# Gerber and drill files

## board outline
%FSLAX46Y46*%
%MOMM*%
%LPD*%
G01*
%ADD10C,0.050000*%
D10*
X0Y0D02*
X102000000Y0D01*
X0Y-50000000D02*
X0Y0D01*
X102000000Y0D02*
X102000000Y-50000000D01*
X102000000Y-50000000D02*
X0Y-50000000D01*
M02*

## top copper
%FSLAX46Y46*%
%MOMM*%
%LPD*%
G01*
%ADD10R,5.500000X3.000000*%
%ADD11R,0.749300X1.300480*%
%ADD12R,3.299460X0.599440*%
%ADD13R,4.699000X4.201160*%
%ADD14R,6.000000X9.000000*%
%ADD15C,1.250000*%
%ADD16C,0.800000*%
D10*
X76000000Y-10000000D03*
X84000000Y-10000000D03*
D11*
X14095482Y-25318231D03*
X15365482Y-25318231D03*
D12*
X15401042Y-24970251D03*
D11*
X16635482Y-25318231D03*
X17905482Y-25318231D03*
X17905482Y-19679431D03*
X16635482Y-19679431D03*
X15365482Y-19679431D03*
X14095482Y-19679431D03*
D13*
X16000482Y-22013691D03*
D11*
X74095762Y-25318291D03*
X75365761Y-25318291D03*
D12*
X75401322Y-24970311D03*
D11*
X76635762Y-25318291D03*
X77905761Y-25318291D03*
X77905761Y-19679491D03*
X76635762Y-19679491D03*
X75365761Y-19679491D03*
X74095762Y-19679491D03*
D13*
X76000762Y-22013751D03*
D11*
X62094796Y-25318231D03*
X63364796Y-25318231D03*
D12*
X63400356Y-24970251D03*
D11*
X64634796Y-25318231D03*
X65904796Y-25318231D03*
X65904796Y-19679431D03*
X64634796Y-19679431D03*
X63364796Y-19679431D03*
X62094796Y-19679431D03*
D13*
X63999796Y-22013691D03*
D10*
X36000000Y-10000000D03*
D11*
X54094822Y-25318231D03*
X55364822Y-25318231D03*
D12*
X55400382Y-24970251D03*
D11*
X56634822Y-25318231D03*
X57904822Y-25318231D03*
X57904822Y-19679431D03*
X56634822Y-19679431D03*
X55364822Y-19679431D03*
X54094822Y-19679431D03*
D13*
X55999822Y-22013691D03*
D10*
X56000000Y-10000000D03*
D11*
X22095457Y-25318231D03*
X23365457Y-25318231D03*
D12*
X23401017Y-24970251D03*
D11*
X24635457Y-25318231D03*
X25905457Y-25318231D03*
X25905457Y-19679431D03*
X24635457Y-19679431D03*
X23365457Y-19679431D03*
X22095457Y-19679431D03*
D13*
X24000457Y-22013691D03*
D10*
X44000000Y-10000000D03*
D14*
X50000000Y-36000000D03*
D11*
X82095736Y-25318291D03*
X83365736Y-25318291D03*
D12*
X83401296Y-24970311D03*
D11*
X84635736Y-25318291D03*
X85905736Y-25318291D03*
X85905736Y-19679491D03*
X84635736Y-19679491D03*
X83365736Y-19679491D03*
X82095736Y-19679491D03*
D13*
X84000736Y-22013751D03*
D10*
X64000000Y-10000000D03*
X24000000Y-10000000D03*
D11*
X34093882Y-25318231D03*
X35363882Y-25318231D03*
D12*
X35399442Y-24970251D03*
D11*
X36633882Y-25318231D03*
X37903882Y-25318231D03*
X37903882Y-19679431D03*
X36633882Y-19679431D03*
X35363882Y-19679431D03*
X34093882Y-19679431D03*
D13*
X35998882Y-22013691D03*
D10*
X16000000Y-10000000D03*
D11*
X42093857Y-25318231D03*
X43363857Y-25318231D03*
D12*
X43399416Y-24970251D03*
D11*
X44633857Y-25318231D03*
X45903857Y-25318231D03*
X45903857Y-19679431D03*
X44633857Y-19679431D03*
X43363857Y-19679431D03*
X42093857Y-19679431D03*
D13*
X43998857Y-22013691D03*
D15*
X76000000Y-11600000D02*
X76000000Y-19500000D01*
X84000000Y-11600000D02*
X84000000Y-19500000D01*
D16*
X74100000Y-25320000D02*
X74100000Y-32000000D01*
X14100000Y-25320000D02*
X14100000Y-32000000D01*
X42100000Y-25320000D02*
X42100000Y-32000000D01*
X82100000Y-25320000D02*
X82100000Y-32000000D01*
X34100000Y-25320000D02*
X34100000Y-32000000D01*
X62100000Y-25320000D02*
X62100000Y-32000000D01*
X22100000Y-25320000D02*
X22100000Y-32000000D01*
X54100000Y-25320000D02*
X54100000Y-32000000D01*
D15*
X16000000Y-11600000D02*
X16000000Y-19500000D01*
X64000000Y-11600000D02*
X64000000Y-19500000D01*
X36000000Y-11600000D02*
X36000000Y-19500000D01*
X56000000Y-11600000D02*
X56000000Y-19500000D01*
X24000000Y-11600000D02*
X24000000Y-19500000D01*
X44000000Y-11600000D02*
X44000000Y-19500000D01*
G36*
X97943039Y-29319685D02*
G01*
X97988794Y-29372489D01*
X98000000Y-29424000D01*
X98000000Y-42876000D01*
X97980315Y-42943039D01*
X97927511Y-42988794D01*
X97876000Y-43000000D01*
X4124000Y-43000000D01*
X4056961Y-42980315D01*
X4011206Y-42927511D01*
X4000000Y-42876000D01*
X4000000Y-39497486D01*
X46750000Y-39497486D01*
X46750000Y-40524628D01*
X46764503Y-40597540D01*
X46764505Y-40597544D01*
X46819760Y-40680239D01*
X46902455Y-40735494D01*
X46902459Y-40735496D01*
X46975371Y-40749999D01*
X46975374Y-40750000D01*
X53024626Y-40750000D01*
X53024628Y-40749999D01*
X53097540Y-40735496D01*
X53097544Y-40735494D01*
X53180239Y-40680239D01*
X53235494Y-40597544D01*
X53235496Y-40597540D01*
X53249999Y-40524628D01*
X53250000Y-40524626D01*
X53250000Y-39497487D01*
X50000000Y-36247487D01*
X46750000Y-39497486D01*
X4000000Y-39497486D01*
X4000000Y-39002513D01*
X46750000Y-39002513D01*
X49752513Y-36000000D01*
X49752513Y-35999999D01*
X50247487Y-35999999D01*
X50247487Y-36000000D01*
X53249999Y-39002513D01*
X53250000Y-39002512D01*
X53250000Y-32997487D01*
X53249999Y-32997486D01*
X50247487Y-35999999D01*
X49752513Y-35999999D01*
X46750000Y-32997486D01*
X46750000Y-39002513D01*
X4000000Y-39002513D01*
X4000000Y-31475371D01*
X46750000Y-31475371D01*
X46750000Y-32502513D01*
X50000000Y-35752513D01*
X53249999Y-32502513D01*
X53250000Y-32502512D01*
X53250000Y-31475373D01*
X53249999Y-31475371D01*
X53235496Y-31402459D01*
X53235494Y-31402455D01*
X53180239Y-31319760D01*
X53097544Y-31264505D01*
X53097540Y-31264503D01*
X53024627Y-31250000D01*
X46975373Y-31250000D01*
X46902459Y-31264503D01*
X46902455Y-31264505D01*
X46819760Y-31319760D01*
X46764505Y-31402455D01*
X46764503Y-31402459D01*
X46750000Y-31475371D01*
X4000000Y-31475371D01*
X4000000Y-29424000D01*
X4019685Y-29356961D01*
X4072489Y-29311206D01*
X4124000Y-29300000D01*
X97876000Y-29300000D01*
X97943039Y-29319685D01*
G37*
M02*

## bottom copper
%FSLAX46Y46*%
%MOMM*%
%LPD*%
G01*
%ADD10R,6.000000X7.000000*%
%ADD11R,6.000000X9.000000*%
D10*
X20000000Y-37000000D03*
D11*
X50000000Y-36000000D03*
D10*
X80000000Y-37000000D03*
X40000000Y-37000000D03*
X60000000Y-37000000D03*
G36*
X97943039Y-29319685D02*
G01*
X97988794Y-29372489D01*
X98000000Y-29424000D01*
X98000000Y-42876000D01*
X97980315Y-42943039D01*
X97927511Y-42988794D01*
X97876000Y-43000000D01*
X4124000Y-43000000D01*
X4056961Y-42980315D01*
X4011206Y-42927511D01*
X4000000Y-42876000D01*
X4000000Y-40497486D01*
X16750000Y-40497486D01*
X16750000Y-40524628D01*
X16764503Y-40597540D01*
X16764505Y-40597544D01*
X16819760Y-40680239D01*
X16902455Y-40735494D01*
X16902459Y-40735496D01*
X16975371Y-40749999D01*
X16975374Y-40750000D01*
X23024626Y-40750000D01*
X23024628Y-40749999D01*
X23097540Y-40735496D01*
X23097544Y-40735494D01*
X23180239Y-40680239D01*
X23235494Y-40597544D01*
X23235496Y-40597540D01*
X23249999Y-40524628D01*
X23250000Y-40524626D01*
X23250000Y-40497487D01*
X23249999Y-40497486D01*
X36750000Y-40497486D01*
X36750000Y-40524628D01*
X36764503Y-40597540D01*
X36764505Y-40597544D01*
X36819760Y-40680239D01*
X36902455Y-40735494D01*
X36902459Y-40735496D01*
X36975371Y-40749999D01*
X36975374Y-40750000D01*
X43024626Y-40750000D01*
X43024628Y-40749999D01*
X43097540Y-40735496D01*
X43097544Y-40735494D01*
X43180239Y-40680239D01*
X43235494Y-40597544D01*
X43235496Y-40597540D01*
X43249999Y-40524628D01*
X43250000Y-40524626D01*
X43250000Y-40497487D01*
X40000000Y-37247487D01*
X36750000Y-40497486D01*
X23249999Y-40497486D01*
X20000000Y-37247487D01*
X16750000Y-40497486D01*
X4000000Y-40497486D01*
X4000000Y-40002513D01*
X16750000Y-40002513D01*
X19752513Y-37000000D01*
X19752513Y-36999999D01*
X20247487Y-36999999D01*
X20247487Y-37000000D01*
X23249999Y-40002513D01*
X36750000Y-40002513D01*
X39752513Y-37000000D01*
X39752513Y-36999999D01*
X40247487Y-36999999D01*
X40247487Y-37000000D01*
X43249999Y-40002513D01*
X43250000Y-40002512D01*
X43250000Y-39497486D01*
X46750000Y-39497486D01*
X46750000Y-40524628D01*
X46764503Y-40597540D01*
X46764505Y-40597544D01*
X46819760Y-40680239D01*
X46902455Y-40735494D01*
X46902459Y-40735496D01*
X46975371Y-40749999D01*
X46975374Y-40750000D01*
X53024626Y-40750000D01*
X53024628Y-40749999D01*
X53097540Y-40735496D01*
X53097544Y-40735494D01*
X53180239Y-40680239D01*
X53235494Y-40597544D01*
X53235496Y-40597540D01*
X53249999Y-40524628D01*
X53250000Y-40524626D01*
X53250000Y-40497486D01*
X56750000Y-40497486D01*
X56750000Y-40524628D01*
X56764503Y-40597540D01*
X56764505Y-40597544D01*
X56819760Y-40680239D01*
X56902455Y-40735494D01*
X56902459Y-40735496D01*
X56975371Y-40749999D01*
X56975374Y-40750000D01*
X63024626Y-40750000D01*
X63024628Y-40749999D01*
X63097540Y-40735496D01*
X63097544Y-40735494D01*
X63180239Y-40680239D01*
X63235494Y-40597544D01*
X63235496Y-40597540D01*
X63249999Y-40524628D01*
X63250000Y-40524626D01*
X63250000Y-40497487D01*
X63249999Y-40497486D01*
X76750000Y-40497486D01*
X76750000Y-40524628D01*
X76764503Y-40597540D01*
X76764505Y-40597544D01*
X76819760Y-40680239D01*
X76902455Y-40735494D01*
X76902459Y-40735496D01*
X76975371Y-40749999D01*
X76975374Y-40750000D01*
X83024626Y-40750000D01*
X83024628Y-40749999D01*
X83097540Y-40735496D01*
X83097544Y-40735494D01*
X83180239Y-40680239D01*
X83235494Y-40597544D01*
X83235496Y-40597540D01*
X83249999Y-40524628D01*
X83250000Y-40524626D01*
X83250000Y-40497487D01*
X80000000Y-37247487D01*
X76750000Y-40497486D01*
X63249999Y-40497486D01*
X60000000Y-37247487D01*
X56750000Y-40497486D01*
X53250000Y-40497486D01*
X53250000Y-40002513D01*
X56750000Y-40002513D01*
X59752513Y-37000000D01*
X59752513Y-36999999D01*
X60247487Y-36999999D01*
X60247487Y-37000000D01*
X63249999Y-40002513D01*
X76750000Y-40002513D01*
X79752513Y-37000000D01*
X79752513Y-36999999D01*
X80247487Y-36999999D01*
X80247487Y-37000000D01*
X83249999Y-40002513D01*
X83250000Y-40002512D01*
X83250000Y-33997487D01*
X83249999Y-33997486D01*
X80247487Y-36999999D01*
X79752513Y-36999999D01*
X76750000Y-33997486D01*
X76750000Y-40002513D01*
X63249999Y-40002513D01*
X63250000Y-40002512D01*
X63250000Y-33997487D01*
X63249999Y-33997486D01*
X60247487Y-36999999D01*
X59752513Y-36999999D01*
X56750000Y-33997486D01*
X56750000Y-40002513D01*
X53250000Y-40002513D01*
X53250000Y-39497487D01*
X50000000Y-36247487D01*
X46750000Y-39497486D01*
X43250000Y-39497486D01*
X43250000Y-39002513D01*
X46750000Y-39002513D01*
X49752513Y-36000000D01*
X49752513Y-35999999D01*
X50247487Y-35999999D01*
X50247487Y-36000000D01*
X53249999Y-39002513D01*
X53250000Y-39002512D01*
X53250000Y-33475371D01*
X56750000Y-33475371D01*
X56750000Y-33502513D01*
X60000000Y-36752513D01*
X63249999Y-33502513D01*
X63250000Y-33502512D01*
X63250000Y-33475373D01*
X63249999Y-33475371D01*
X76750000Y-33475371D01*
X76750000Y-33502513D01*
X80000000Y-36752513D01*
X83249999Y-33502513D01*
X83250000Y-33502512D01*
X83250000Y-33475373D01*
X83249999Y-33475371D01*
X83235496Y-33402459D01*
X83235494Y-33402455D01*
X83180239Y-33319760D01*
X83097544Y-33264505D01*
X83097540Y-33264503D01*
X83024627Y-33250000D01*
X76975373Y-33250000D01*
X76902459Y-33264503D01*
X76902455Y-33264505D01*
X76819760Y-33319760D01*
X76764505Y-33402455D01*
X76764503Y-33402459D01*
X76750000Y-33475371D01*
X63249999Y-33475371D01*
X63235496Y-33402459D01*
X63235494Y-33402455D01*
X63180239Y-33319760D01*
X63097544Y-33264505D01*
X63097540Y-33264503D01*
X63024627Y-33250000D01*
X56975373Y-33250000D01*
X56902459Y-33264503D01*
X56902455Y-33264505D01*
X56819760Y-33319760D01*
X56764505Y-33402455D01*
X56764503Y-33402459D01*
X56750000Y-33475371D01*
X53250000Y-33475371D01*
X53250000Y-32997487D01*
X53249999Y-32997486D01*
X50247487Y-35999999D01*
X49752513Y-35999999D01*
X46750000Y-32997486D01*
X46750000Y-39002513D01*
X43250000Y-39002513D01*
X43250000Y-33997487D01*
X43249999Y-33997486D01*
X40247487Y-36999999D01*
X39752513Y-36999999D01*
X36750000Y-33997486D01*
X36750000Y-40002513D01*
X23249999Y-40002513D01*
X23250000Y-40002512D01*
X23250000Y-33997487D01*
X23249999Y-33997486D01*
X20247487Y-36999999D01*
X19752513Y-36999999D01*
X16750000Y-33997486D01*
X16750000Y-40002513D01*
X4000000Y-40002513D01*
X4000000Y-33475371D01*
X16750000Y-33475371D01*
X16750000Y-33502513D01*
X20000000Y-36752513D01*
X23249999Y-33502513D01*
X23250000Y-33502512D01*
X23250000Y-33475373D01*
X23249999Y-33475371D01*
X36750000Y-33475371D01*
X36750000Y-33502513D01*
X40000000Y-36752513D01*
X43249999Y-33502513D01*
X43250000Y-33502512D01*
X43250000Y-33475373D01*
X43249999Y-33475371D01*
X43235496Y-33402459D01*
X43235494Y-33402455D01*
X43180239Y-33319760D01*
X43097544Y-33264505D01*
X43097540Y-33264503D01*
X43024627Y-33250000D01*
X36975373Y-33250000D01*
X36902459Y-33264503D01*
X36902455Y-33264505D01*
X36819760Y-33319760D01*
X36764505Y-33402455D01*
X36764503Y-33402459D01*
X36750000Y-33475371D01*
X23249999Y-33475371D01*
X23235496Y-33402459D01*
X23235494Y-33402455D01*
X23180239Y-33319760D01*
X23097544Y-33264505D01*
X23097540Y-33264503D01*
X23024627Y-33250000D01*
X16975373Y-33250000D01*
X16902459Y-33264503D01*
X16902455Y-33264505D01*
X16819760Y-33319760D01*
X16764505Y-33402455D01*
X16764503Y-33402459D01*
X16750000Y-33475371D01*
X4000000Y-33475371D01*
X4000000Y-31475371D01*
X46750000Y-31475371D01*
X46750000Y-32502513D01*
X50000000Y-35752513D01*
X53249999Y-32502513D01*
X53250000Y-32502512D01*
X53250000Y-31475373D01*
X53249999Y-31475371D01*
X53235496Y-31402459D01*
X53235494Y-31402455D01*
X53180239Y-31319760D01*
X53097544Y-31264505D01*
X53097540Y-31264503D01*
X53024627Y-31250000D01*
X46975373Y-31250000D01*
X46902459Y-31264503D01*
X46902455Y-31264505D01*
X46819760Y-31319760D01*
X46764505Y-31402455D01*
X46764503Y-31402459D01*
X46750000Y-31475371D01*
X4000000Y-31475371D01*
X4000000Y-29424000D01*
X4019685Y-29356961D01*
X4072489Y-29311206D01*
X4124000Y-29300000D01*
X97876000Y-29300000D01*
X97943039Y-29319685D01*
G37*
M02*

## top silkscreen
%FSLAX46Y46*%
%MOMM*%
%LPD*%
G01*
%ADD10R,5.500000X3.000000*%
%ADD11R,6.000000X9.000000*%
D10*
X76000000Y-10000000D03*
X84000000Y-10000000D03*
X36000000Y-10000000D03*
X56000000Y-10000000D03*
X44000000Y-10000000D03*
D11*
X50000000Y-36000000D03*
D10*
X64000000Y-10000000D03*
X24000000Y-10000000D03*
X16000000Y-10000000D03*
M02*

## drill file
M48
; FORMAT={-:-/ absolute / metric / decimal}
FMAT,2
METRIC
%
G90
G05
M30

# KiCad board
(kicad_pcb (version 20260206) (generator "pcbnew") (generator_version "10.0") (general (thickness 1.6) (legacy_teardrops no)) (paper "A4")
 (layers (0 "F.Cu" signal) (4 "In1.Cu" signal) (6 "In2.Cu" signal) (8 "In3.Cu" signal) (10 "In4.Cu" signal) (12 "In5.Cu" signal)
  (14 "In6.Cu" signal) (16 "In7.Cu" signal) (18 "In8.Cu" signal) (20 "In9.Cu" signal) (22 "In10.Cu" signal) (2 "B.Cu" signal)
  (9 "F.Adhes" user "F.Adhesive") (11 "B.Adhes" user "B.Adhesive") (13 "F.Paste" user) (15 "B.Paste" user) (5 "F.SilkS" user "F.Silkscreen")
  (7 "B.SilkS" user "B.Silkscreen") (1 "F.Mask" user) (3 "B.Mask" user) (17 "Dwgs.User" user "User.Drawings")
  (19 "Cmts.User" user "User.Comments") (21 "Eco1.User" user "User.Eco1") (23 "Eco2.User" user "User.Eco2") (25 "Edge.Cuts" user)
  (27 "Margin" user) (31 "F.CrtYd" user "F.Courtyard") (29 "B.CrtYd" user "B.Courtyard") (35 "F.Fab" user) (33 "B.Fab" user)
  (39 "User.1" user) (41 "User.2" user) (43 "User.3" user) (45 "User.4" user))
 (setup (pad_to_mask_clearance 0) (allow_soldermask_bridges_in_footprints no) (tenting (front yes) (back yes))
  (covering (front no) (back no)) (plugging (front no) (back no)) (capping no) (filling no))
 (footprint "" (layer "F.Cu") (at 76 10)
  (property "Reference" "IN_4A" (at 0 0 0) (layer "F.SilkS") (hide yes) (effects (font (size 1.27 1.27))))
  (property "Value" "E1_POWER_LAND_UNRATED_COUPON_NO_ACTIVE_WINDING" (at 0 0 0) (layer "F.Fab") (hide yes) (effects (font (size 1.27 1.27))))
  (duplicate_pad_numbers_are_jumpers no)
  (pad "1" smd rect (at 0 0) (size 5.5 3)
   (layers "F.Cu" "F.Mask" "F.SilkS" "F.Adhes" "F.Paste" "F.CrtYd" "F.Fab") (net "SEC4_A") (thermal_bridge_angle 45)))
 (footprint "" (layer "F.Cu") (at 84 10)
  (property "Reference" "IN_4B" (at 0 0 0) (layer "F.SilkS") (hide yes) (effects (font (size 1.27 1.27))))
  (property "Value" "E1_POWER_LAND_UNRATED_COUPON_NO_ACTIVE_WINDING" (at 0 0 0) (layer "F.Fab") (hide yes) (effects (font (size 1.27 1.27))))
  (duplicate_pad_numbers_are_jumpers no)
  (pad "1" smd rect (at 0 0) (size 5.5 3)
   (layers "F.Cu" "F.Mask" "F.SilkS" "F.Adhes" "F.Paste" "F.CrtYd" "F.Fab") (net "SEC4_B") (thermal_bridge_angle 45)))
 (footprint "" (layer "F.Cu") (at 16 22.5)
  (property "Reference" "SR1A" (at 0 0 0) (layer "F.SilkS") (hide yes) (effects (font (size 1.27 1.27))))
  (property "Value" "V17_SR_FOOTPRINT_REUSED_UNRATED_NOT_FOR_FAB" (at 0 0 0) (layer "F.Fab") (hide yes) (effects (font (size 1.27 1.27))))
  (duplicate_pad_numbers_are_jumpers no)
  (pad "1" smd rect (at -1.904518 2.818231 90) (size 1.30048 0.7493) (layers "F.Cu" "F.Mask" "F.Paste") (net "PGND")
   (thermal_bridge_angle 45))
  (pad "2" smd rect (at -0.634518 2.818231 90) (size 1.30048 0.7493) (layers "F.Cu" "F.Mask" "F.Paste") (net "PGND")
   (thermal_bridge_angle 45))
  (pad "3" smd rect (at -0.598958 2.470251 90) (size 0.59944 3.29946) (layers "F.Cu" "F.Mask" "F.Paste") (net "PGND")
   (thermal_bridge_angle 45))
  (pad "3" smd rect (at 0.635482 2.818231 90) (size 1.30048 0.7493) (layers "F.Cu" "F.Mask" "F.Paste") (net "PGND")
   (thermal_bridge_angle 45))
  (pad "4" smd rect (at 1.905482 2.818231 90) (size 1.30048 0.7493) (layers "F.Cu" "F.Mask" "F.Paste") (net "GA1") (thermal_bridge_angle 45))
  (pad "5" smd rect (at 1.905482 -2.820569 270) (size 1.30048 0.7493) (layers "F.Cu" "F.Mask" "F.Paste") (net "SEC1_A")
   (thermal_bridge_angle 45))
  (pad "6" smd rect (at 0.635482 -2.820569 270) (size 1.30048 0.7493) (layers "F.Cu" "F.Mask" "F.Paste") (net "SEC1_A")
   (thermal_bridge_angle 45))
  (pad "7" smd rect (at -0.634518 -2.820569 270) (size 1.30048 0.7493) (layers "F.Cu" "F.Mask" "F.Paste") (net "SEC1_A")
   (thermal_bridge_angle 45))
  (pad "8" smd rect (at -1.904518 -2.820569 270) (size 1.30048 0.7493) (layers "F.Cu" "F.Mask" "F.Paste") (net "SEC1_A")
   (thermal_bridge_angle 45))
  (pad "8" smd rect (at 0.000482 -0.486309) (size 4.699 4.20116) (layers "F.Cu" "F.Mask" "F.Paste") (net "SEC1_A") (thermal_bridge_angle 45)))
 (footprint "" (layer "F.Cu") (at 76 22.5)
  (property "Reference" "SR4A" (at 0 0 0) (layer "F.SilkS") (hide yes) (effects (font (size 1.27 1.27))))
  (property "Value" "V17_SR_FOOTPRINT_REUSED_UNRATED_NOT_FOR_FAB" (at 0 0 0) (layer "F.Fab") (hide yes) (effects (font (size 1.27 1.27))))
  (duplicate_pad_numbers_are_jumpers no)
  (pad "1" smd rect (at -1.904238 2.818291 90) (size 1.30048 0.7493) (layers "F.Cu" "F.Mask" "F.Paste") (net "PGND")
   (thermal_bridge_angle 45))
  (pad "2" smd rect (at -0.634239 2.818291 90) (size 1.30048 0.7493) (layers "F.Cu" "F.Mask" "F.Paste") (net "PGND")
   (thermal_bridge_angle 45))
  (pad "3" smd rect (at -0.598678 2.470311 90) (size 0.59944 3.29946) (layers "F.Cu" "F.Mask" "F.Paste") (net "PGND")
   (thermal_bridge_angle 45))
  (pad "3" smd rect (at 0.635762 2.818291 90) (size 1.30048 0.7493) (layers "F.Cu" "F.Mask" "F.Paste") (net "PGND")
   (thermal_bridge_angle 45))
  (pad "4" smd rect (at 1.905761 2.818291 90) (size 1.30048 0.7493) (layers "F.Cu" "F.Mask" "F.Paste") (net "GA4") (thermal_bridge_angle 45))
  (pad "5" smd rect (at 1.905761 -2.820509 270) (size 1.30048 0.7493) (layers "F.Cu" "F.Mask" "F.Paste") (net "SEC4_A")
   (thermal_bridge_angle 45))
  (pad "6" smd rect (at 0.635762 -2.820509 270) (size 1.30048 0.7493) (layers "F.Cu" "F.Mask" "F.Paste") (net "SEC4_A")
   (thermal_bridge_angle 45))
  (pad "7" smd rect (at -0.634239 -2.820509 270) (size 1.30048 0.7493) (layers "F.Cu" "F.Mask" "F.Paste") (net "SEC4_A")
   (thermal_bridge_angle 45))
  (pad "8" smd rect (at -1.904238 -2.820509 270) (size 1.30048 0.7493) (layers "F.Cu" "F.Mask" "F.Paste") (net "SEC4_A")
   (thermal_bridge_angle 45))
  (pad "8" smd rect (at 0.000762 -0.486249) (size 4.699 4.20116) (layers "F.Cu" "F.Mask" "F.Paste") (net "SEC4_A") (thermal_bridge_angle 45)))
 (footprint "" (layer "F.Cu") (at 20 37)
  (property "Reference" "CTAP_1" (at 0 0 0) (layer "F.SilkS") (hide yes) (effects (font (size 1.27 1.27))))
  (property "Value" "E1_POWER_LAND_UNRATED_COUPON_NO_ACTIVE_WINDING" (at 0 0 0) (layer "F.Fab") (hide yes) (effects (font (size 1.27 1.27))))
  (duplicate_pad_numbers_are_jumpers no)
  (pad "1" smd rect (at 0 0) (size 6 7)
   (layers "B.Cu" "B.Mask" "B.SilkS" "B.Adhes" "B.Paste" "B.CrtYd" "B.Fab") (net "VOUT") (thermal_bridge_angle 45)))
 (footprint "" (layer "F.Cu") (at 64 22.5)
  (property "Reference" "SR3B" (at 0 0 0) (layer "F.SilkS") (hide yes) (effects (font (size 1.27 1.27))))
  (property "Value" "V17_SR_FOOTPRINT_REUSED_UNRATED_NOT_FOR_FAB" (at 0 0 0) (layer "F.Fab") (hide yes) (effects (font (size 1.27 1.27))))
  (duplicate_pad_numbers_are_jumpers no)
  (pad "1" smd rect (at -1.905204 2.818231 90) (size 1.30048 0.7493) (layers "F.Cu" "F.Mask" "F.Paste") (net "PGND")
   (thermal_bridge_angle 45))
  (pad "2" smd rect (at -0.635204 2.818231 90) (size 1.30048 0.7493) (layers "F.Cu" "F.Mask" "F.Paste") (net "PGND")
   (thermal_bridge_angle 45))
  (pad "3" smd rect (at -0.599644 2.470251 90) (size 0.59944 3.29946) (layers "F.Cu" "F.Mask" "F.Paste") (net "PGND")
   (thermal_bridge_angle 45))
  (pad "3" smd rect (at 0.634796 2.818231 90) (size 1.30048 0.7493) (layers "F.Cu" "F.Mask" "F.Paste") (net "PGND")
   (thermal_bridge_angle 45))
  (pad "4" smd rect (at 1.904796 2.818231 90) (size 1.30048 0.7493) (layers "F.Cu" "F.Mask" "F.Paste") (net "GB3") (thermal_bridge_angle 45))
  (pad "5" smd rect (at 1.904796 -2.820569 270) (size 1.30048 0.7493) (layers "F.Cu" "F.Mask" "F.Paste") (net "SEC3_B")
   (thermal_bridge_angle 45))
  (pad "6" smd rect (at 0.634796 -2.820569 270) (size 1.30048 0.7493) (layers "F.Cu" "F.Mask" "F.Paste") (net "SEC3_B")
   (thermal_bridge_angle 45))
  (pad "7" smd rect (at -0.635204 -2.820569 270) (size 1.30048 0.7493) (layers "F.Cu" "F.Mask" "F.Paste") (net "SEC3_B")
   (thermal_bridge_angle 45))
  (pad "8" smd rect (at -1.905204 -2.820569 270) (size 1.30048 0.7493) (layers "F.Cu" "F.Mask" "F.Paste") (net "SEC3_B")
   (thermal_bridge_angle 45))
  (pad "8" smd rect (at -0.000204 -0.486309) (size 4.699 4.20116) (layers "F.Cu" "F.Mask" "F.Paste") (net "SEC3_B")
   (thermal_bridge_angle 45)))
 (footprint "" (layer "F.Cu") (at 36 10)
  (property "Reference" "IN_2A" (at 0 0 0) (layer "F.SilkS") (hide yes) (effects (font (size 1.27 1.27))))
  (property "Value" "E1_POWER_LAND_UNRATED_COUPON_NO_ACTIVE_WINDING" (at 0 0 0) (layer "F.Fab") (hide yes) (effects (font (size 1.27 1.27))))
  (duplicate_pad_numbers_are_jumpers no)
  (pad "1" smd rect (at 0 0) (size 5.5 3)
   (layers "F.Cu" "F.Mask" "F.SilkS" "F.Adhes" "F.Paste" "F.CrtYd" "F.Fab") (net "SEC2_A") (thermal_bridge_angle 45)))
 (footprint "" (layer "F.Cu") (at 56 22.5)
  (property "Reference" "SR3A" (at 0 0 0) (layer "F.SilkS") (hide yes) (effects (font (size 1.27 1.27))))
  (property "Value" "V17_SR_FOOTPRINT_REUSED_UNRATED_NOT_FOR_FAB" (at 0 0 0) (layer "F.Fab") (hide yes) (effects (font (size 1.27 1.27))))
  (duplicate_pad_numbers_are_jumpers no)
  (pad "1" smd rect (at -1.905178 2.818231 90) (size 1.30048 0.7493) (layers "F.Cu" "F.Mask" "F.Paste") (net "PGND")
   (thermal_bridge_angle 45))
  (pad "2" smd rect (at -0.635178 2.818231 90) (size 1.30048 0.7493) (layers "F.Cu" "F.Mask" "F.Paste") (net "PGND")
   (thermal_bridge_angle 45))
  (pad "3" smd rect (at -0.599618 2.470251 90) (size 0.59944 3.29946) (layers "F.Cu" "F.Mask" "F.Paste") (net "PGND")
   (thermal_bridge_angle 45))
  (pad "3" smd rect (at 0.634822 2.818231 90) (size 1.30048 0.7493) (layers "F.Cu" "F.Mask" "F.Paste") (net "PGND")
   (thermal_bridge_angle 45))
  (pad "4" smd rect (at 1.904822 2.818231 90) (size 1.30048 0.7493) (layers "F.Cu" "F.Mask" "F.Paste") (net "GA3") (thermal_bridge_angle 45))
  (pad "5" smd rect (at 1.904822 -2.820569 270) (size 1.30048 0.7493) (layers "F.Cu" "F.Mask" "F.Paste") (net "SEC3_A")
   (thermal_bridge_angle 45))
  (pad "6" smd rect (at 0.634822 -2.820569 270) (size 1.30048 0.7493) (layers "F.Cu" "F.Mask" "F.Paste") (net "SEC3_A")
   (thermal_bridge_angle 45))
  (pad "7" smd rect (at -0.635178 -2.820569 270) (size 1.30048 0.7493) (layers "F.Cu" "F.Mask" "F.Paste") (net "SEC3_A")
   (thermal_bridge_angle 45))
  (pad "8" smd rect (at -1.905178 -2.820569 270) (size 1.30048 0.7493) (layers "F.Cu" "F.Mask" "F.Paste") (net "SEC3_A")
   (thermal_bridge_angle 45))
  (pad "8" smd rect (at -0.000178 -0.486309) (size 4.699 4.20116) (layers "F.Cu" "F.Mask" "F.Paste") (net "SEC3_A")
   (thermal_bridge_angle 45)))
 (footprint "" (layer "F.Cu") (at 56 10)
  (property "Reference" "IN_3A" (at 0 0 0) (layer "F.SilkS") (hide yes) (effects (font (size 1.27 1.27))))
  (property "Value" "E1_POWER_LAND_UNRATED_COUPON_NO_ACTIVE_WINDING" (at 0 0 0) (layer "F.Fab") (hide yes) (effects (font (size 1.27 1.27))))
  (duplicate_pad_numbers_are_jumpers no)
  (pad "1" smd rect (at 0 0) (size 5.5 3)
   (layers "F.Cu" "F.Mask" "F.SilkS" "F.Adhes" "F.Paste" "F.CrtYd" "F.Fab") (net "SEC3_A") (thermal_bridge_angle 45)))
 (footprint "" (layer "F.Cu") (at 50 36)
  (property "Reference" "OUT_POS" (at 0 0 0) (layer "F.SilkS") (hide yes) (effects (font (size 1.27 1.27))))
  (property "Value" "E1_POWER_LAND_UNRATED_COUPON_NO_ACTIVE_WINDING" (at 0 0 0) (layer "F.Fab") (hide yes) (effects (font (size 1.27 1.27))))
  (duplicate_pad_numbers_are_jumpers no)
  (pad "1" smd rect (at 0 0) (size 6 9)
   (layers "B.Cu" "B.Mask" "B.SilkS" "B.Adhes" "B.Paste" "B.CrtYd" "B.Fab") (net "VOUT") (thermal_bridge_angle 45)))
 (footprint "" (layer "F.Cu") (at 24 22.5)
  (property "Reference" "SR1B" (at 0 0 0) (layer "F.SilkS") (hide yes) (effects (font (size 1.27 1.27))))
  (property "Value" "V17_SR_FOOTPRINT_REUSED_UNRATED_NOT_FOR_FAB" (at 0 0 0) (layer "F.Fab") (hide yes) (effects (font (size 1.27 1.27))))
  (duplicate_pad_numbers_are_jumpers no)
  (pad "1" smd rect (at -1.904543 2.818231 90) (size 1.30048 0.7493) (layers "F.Cu" "F.Mask" "F.Paste") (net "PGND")
   (thermal_bridge_angle 45))
  (pad "2" smd rect (at -0.634543 2.818231 90) (size 1.30048 0.7493) (layers "F.Cu" "F.Mask" "F.Paste") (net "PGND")
   (thermal_bridge_angle 45))
  (pad "3" smd rect (at -0.598983 2.470251 90) (size 0.59944 3.29946) (layers "F.Cu" "F.Mask" "F.Paste") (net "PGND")
   (thermal_bridge_angle 45))
  (pad "3" smd rect (at 0.635457 2.818231 90) (size 1.30048 0.7493) (layers "F.Cu" "F.Mask" "F.Paste") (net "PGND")
   (thermal_bridge_angle 45))
  (pad "4" smd rect (at 1.905457 2.818231 90) (size 1.30048 0.7493) (layers "F.Cu" "F.Mask" "F.Paste") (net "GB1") (thermal_bridge_angle 45))
  (pad "5" smd rect (at 1.905457 -2.820569 270) (size 1.30048 0.7493) (layers "F.Cu" "F.Mask" "F.Paste") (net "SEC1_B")
   (thermal_bridge_angle 45))
  (pad "6" smd rect (at 0.635457 -2.820569 270) (size 1.30048 0.7493) (layers "F.Cu" "F.Mask" "F.Paste") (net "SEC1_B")
   (thermal_bridge_angle 45))
  (pad "7" smd rect (at -0.634543 -2.820569 270) (size 1.30048 0.7493) (layers "F.Cu" "F.Mask" "F.Paste") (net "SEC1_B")
   (thermal_bridge_angle 45))
  (pad "8" smd rect (at -1.904543 -2.820569 270) (size 1.30048 0.7493) (layers "F.Cu" "F.Mask" "F.Paste") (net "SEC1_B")
   (thermal_bridge_angle 45))
  (pad "8" smd rect (at 0.000457 -0.486309) (size 4.699 4.20116) (layers "F.Cu" "F.Mask" "F.Paste") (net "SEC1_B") (thermal_bridge_angle 45)))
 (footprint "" (layer "F.Cu") (at 80 37)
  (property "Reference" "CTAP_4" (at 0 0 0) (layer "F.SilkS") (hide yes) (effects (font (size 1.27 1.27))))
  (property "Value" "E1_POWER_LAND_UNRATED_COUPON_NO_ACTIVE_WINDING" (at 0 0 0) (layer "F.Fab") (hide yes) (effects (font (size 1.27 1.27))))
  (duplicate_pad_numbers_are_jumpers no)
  (pad "1" smd rect (at 0 0) (size 6 7)
   (layers "B.Cu" "B.Mask" "B.SilkS" "B.Adhes" "B.Paste" "B.CrtYd" "B.Fab") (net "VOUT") (thermal_bridge_angle 45)))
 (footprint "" (layer "F.Cu") (at 44 10)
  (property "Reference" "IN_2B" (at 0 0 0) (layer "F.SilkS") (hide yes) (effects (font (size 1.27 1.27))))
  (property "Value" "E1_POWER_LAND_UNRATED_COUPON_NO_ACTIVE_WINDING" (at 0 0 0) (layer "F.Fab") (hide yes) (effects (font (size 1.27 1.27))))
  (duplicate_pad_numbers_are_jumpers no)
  (pad "1" smd rect (at 0 0) (size 5.5 3)
   (layers "F.Cu" "F.Mask" "F.SilkS" "F.Adhes" "F.Paste" "F.CrtYd" "F.Fab") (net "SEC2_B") (thermal_bridge_angle 45)))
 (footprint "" (layer "F.Cu") (at 40 37)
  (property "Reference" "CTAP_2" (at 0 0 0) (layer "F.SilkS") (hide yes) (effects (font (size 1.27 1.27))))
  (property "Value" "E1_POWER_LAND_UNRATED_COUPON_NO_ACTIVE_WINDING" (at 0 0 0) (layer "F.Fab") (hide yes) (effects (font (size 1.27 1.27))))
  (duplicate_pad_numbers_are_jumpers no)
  (pad "1" smd rect (at 0 0) (size 6 7)
   (layers "B.Cu" "B.Mask" "B.SilkS" "B.Adhes" "B.Paste" "B.CrtYd" "B.Fab") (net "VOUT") (thermal_bridge_angle 45)))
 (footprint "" (layer "F.Cu") (at 50 36)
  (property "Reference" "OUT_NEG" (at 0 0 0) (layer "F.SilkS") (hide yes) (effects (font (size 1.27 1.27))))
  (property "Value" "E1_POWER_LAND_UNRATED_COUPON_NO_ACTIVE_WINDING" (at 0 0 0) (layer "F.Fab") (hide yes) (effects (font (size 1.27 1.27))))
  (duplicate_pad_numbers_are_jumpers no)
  (pad "1" smd rect (at 0 0) (size 6 9)
   (layers "F.Cu" "F.Mask" "F.SilkS" "F.Adhes" "F.Paste" "F.CrtYd" "F.Fab") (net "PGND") (thermal_bridge_angle 45)))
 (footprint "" (layer "F.Cu") (at 84 22.5)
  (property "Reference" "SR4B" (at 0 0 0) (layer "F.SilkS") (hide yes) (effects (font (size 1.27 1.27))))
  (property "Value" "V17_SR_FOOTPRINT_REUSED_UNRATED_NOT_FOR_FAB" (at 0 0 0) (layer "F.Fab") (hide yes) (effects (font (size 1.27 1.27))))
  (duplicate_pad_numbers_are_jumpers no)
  (pad "1" smd rect (at -1.904264 2.818291 90) (size 1.30048 0.7493) (layers "F.Cu" "F.Mask" "F.Paste") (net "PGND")
   (thermal_bridge_angle 45))
  (pad "2" smd rect (at -0.634264 2.818291 90) (size 1.30048 0.7493) (layers "F.Cu" "F.Mask" "F.Paste") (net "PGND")
   (thermal_bridge_angle 45))
  (pad "3" smd rect (at -0.598704 2.470311 90) (size 0.59944 3.29946) (layers "F.Cu" "F.Mask" "F.Paste") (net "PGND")
   (thermal_bridge_angle 45))
  (pad "3" smd rect (at 0.635736 2.818291 90) (size 1.30048 0.7493) (layers "F.Cu" "F.Mask" "F.Paste") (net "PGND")
   (thermal_bridge_angle 45))
  (pad "4" smd rect (at 1.905736 2.818291 90) (size 1.30048 0.7493) (layers "F.Cu" "F.Mask" "F.Paste") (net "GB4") (thermal_bridge_angle 45))
  (pad "5" smd rect (at 1.905736 -2.820509 270) (size 1.30048 0.7493) (layers "F.Cu" "F.Mask" "F.Paste") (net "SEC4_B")
   (thermal_bridge_angle 45))
  (pad "6" smd rect (at 0.635736 -2.820509 270) (size 1.30048 0.7493) (layers "F.Cu" "F.Mask" "F.Paste") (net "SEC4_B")
   (thermal_bridge_angle 45))
  (pad "7" smd rect (at -0.634264 -2.820509 270) (size 1.30048 0.7493) (layers "F.Cu" "F.Mask" "F.Paste") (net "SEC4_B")
   (thermal_bridge_angle 45))
  (pad "8" smd rect (at -1.904264 -2.820509 270) (size 1.30048 0.7493) (layers "F.Cu" "F.Mask" "F.Paste") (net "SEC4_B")
   (thermal_bridge_angle 45))
  (pad "8" smd rect (at 0.000736 -0.486249) (size 4.699 4.20116) (layers "F.Cu" "F.Mask" "F.Paste") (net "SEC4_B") (thermal_bridge_angle 45)))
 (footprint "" (layer "F.Cu") (at 64 10)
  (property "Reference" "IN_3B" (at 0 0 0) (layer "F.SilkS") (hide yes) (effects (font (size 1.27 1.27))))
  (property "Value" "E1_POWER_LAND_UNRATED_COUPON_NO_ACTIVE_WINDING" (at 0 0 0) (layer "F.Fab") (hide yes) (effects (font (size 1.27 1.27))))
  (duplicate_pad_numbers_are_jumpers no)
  (pad "1" smd rect (at 0 0) (size 5.5 3)
   (layers "F.Cu" "F.Mask" "F.SilkS" "F.Adhes" "F.Paste" "F.CrtYd" "F.Fab") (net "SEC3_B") (thermal_bridge_angle 45)))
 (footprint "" (layer "F.Cu") (at 24 10)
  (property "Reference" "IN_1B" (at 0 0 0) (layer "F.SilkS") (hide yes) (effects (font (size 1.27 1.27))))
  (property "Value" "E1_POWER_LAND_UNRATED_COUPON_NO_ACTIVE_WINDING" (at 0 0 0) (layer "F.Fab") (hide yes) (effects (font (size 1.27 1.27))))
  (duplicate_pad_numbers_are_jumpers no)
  (pad "1" smd rect (at 0 0) (size 5.5 3)
   (layers "F.Cu" "F.Mask" "F.SilkS" "F.Adhes" "F.Paste" "F.CrtYd" "F.Fab") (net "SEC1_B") (thermal_bridge_angle 45)))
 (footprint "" (layer "F.Cu") (at 36 22.5)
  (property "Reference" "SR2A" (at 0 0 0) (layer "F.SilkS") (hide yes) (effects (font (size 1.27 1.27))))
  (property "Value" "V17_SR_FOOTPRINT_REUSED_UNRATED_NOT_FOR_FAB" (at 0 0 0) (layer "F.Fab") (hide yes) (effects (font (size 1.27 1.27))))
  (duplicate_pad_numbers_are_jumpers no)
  (pad "1" smd rect (at -1.906118 2.818231 90) (size 1.30048 0.7493) (layers "F.Cu" "F.Mask" "F.Paste") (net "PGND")
   (thermal_bridge_angle 45))
  (pad "2" smd rect (at -0.636118 2.818231 90) (size 1.30048 0.7493) (layers "F.Cu" "F.Mask" "F.Paste") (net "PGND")
   (thermal_bridge_angle 45))
  (pad "3" smd rect (at -0.600558 2.470251 90) (size 0.59944 3.29946) (layers "F.Cu" "F.Mask" "F.Paste") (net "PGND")
   (thermal_bridge_angle 45))
  (pad "3" smd rect (at 0.633882 2.818231 90) (size 1.30048 0.7493) (layers "F.Cu" "F.Mask" "F.Paste") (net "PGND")
   (thermal_bridge_angle 45))
  (pad "4" smd rect (at 1.903882 2.818231 90) (size 1.30048 0.7493) (layers "F.Cu" "F.Mask" "F.Paste") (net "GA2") (thermal_bridge_angle 45))
  (pad "5" smd rect (at 1.903882 -2.820569 270) (size 1.30048 0.7493) (layers "F.Cu" "F.Mask" "F.Paste") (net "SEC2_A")
   (thermal_bridge_angle 45))
  (pad "6" smd rect (at 0.633882 -2.820569 270) (size 1.30048 0.7493) (layers "F.Cu" "F.Mask" "F.Paste") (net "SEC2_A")
   (thermal_bridge_angle 45))
  (pad "7" smd rect (at -0.636118 -2.820569 270) (size 1.30048 0.7493) (layers "F.Cu" "F.Mask" "F.Paste") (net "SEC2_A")
   (thermal_bridge_angle 45))
  (pad "8" smd rect (at -1.906118 -2.820569 270) (size 1.30048 0.7493) (layers "F.Cu" "F.Mask" "F.Paste") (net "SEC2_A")
   (thermal_bridge_angle 45))
  (pad "8" smd rect (at -0.001118 -0.486309) (size 4.699 4.20116) (layers "F.Cu" "F.Mask" "F.Paste") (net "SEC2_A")
   (thermal_bridge_angle 45)))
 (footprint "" (layer "F.Cu") (at 16 10)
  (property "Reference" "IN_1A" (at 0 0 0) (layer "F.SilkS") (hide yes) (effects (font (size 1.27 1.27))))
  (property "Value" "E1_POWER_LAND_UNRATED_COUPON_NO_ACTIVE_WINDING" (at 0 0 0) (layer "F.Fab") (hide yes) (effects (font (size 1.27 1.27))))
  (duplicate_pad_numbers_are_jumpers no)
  (pad "1" smd rect (at 0 0) (size 5.5 3)
   (layers "F.Cu" "F.Mask" "F.SilkS" "F.Adhes" "F.Paste" "F.CrtYd" "F.Fab") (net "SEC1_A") (thermal_bridge_angle 45)))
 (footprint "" (layer "F.Cu") (at 60 37)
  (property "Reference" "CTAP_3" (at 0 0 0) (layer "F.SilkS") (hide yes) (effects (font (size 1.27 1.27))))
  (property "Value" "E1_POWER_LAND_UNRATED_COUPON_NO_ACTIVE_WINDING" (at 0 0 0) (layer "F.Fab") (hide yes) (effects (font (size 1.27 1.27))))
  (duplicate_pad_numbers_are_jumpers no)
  (pad "1" smd rect (at 0 0) (size 6 7)
   (layers "B.Cu" "B.Mask" "B.SilkS" "B.Adhes" "B.Paste" "B.CrtYd" "B.Fab") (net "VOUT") (thermal_bridge_angle 45)))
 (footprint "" (layer "F.Cu") (at 44 22.5)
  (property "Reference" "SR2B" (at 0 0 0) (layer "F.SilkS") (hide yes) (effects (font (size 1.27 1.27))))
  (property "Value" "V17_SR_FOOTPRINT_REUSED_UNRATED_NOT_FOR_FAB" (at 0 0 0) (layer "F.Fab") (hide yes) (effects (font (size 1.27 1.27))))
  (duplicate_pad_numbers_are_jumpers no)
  (pad "1" smd rect (at -1.906143 2.818231 90) (size 1.30048 0.7493) (layers "F.Cu" "F.Mask" "F.Paste") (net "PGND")
   (thermal_bridge_angle 45))
  (pad "2" smd rect (at -0.636143 2.818231 90) (size 1.30048 0.7493) (layers "F.Cu" "F.Mask" "F.Paste") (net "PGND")
   (thermal_bridge_angle 45))
  (pad "3" smd rect (at -0.600584 2.470251 90) (size 0.59944 3.29946) (layers "F.Cu" "F.Mask" "F.Paste") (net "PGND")
   (thermal_bridge_angle 45))
  (pad "3" smd rect (at 0.633857 2.818231 90) (size 1.30048 0.7493) (layers "F.Cu" "F.Mask" "F.Paste") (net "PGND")
   (thermal_bridge_angle 45))
  (pad "4" smd rect (at 1.903857 2.818231 90) (size 1.30048 0.7493) (layers "F.Cu" "F.Mask" "F.Paste") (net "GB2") (thermal_bridge_angle 45))
  (pad "5" smd rect (at 1.903857 -2.820569 270) (size 1.30048 0.7493) (layers "F.Cu" "F.Mask" "F.Paste") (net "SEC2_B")
   (thermal_bridge_angle 45))
  (pad "6" smd rect (at 0.633857 -2.820569 270) (size 1.30048 0.7493) (layers "F.Cu" "F.Mask" "F.Paste") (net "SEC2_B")
   (thermal_bridge_angle 45))
  (pad "7" smd rect (at -0.636143 -2.820569 270) (size 1.30048 0.7493) (layers "F.Cu" "F.Mask" "F.Paste") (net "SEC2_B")
   (thermal_bridge_angle 45))
  (pad "8" smd rect (at -1.906143 -2.820569 270) (size 1.30048 0.7493) (layers "F.Cu" "F.Mask" "F.Paste") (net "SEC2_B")
   (thermal_bridge_angle 45))
  (pad "8" smd rect (at -0.001143 -0.486309) (size 4.699 4.20116) (layers "F.Cu" "F.Mask" "F.Paste") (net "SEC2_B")
   (thermal_bridge_angle 45)))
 (gr_line (start 0 0) (end 102 0) (stroke (width 0.05) (type default)) (layer "Edge.Cuts"))
 (gr_line (start 0 50) (end 0 0) (stroke (width 0.05) (type default)) (layer "Edge.Cuts"))
 (gr_line (start 102 0) (end 102 50) (stroke (width 0.05) (type default)) (layer "Edge.Cuts"))
 (gr_line (start 102 50) (end 0 50) (stroke (width 0.05) (type default)) (layer "Edge.Cuts"))
 (segment (start 76 11.6) (end 76 19.5) (width 1.25) (layer "F.Cu") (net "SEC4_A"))
 (segment (start 84 11.6) (end 84 19.5) (width 1.25) (layer "F.Cu") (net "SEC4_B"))
 (segment (start 74.1 25.32) (end 74.1 32) (width 0.8) (layer "F.Cu") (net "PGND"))
 (segment (start 14.1 25.32) (end 14.1 32) (width 0.8) (layer "F.Cu") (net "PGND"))
 (segment (start 42.1 25.32) (end 42.1 32) (width 0.8) (layer "F.Cu") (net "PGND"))
 (segment (start 82.1 25.32) (end 82.1 32) (width 0.8) (layer "F.Cu") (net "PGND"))
 (segment (start 34.1 25.32) (end 34.1 32) (width 0.8) (layer "F.Cu") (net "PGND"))
 (segment (start 62.1 25.32) (end 62.1 32) (width 0.8) (layer "F.Cu") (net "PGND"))
 (segment (start 22.1 25.32) (end 22.1 32) (width 0.8) (layer "F.Cu") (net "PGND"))
 (segment (start 54.1 25.32) (end 54.1 32) (width 0.8) (layer "F.Cu") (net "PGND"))
 (segment (start 16 11.6) (end 16 19.5) (width 1.25) (layer "F.Cu") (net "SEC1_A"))
 (segment (start 64 11.6) (end 64 19.5) (width 1.25) (layer "F.Cu") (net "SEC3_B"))
 (segment (start 36 11.6) (end 36 19.5) (width 1.25) (layer "F.Cu") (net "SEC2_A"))
 (segment (start 56 11.6) (end 56 19.5) (width 1.25) (layer "F.Cu") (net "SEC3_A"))
 (segment (start 24 11.6) (end 24 19.5) (width 1.25) (layer "F.Cu") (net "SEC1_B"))
 (segment (start 44 11.6) (end 44 19.5) (width 1.25) (layer "F.Cu") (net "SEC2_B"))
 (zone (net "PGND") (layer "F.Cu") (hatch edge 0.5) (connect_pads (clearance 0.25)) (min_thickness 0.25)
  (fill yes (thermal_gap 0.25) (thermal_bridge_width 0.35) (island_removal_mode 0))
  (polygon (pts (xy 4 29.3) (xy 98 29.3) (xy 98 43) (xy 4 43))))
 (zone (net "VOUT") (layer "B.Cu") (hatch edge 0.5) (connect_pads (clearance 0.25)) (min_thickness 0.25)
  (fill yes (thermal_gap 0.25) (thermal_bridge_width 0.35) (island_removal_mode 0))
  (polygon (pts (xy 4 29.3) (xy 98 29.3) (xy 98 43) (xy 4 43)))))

